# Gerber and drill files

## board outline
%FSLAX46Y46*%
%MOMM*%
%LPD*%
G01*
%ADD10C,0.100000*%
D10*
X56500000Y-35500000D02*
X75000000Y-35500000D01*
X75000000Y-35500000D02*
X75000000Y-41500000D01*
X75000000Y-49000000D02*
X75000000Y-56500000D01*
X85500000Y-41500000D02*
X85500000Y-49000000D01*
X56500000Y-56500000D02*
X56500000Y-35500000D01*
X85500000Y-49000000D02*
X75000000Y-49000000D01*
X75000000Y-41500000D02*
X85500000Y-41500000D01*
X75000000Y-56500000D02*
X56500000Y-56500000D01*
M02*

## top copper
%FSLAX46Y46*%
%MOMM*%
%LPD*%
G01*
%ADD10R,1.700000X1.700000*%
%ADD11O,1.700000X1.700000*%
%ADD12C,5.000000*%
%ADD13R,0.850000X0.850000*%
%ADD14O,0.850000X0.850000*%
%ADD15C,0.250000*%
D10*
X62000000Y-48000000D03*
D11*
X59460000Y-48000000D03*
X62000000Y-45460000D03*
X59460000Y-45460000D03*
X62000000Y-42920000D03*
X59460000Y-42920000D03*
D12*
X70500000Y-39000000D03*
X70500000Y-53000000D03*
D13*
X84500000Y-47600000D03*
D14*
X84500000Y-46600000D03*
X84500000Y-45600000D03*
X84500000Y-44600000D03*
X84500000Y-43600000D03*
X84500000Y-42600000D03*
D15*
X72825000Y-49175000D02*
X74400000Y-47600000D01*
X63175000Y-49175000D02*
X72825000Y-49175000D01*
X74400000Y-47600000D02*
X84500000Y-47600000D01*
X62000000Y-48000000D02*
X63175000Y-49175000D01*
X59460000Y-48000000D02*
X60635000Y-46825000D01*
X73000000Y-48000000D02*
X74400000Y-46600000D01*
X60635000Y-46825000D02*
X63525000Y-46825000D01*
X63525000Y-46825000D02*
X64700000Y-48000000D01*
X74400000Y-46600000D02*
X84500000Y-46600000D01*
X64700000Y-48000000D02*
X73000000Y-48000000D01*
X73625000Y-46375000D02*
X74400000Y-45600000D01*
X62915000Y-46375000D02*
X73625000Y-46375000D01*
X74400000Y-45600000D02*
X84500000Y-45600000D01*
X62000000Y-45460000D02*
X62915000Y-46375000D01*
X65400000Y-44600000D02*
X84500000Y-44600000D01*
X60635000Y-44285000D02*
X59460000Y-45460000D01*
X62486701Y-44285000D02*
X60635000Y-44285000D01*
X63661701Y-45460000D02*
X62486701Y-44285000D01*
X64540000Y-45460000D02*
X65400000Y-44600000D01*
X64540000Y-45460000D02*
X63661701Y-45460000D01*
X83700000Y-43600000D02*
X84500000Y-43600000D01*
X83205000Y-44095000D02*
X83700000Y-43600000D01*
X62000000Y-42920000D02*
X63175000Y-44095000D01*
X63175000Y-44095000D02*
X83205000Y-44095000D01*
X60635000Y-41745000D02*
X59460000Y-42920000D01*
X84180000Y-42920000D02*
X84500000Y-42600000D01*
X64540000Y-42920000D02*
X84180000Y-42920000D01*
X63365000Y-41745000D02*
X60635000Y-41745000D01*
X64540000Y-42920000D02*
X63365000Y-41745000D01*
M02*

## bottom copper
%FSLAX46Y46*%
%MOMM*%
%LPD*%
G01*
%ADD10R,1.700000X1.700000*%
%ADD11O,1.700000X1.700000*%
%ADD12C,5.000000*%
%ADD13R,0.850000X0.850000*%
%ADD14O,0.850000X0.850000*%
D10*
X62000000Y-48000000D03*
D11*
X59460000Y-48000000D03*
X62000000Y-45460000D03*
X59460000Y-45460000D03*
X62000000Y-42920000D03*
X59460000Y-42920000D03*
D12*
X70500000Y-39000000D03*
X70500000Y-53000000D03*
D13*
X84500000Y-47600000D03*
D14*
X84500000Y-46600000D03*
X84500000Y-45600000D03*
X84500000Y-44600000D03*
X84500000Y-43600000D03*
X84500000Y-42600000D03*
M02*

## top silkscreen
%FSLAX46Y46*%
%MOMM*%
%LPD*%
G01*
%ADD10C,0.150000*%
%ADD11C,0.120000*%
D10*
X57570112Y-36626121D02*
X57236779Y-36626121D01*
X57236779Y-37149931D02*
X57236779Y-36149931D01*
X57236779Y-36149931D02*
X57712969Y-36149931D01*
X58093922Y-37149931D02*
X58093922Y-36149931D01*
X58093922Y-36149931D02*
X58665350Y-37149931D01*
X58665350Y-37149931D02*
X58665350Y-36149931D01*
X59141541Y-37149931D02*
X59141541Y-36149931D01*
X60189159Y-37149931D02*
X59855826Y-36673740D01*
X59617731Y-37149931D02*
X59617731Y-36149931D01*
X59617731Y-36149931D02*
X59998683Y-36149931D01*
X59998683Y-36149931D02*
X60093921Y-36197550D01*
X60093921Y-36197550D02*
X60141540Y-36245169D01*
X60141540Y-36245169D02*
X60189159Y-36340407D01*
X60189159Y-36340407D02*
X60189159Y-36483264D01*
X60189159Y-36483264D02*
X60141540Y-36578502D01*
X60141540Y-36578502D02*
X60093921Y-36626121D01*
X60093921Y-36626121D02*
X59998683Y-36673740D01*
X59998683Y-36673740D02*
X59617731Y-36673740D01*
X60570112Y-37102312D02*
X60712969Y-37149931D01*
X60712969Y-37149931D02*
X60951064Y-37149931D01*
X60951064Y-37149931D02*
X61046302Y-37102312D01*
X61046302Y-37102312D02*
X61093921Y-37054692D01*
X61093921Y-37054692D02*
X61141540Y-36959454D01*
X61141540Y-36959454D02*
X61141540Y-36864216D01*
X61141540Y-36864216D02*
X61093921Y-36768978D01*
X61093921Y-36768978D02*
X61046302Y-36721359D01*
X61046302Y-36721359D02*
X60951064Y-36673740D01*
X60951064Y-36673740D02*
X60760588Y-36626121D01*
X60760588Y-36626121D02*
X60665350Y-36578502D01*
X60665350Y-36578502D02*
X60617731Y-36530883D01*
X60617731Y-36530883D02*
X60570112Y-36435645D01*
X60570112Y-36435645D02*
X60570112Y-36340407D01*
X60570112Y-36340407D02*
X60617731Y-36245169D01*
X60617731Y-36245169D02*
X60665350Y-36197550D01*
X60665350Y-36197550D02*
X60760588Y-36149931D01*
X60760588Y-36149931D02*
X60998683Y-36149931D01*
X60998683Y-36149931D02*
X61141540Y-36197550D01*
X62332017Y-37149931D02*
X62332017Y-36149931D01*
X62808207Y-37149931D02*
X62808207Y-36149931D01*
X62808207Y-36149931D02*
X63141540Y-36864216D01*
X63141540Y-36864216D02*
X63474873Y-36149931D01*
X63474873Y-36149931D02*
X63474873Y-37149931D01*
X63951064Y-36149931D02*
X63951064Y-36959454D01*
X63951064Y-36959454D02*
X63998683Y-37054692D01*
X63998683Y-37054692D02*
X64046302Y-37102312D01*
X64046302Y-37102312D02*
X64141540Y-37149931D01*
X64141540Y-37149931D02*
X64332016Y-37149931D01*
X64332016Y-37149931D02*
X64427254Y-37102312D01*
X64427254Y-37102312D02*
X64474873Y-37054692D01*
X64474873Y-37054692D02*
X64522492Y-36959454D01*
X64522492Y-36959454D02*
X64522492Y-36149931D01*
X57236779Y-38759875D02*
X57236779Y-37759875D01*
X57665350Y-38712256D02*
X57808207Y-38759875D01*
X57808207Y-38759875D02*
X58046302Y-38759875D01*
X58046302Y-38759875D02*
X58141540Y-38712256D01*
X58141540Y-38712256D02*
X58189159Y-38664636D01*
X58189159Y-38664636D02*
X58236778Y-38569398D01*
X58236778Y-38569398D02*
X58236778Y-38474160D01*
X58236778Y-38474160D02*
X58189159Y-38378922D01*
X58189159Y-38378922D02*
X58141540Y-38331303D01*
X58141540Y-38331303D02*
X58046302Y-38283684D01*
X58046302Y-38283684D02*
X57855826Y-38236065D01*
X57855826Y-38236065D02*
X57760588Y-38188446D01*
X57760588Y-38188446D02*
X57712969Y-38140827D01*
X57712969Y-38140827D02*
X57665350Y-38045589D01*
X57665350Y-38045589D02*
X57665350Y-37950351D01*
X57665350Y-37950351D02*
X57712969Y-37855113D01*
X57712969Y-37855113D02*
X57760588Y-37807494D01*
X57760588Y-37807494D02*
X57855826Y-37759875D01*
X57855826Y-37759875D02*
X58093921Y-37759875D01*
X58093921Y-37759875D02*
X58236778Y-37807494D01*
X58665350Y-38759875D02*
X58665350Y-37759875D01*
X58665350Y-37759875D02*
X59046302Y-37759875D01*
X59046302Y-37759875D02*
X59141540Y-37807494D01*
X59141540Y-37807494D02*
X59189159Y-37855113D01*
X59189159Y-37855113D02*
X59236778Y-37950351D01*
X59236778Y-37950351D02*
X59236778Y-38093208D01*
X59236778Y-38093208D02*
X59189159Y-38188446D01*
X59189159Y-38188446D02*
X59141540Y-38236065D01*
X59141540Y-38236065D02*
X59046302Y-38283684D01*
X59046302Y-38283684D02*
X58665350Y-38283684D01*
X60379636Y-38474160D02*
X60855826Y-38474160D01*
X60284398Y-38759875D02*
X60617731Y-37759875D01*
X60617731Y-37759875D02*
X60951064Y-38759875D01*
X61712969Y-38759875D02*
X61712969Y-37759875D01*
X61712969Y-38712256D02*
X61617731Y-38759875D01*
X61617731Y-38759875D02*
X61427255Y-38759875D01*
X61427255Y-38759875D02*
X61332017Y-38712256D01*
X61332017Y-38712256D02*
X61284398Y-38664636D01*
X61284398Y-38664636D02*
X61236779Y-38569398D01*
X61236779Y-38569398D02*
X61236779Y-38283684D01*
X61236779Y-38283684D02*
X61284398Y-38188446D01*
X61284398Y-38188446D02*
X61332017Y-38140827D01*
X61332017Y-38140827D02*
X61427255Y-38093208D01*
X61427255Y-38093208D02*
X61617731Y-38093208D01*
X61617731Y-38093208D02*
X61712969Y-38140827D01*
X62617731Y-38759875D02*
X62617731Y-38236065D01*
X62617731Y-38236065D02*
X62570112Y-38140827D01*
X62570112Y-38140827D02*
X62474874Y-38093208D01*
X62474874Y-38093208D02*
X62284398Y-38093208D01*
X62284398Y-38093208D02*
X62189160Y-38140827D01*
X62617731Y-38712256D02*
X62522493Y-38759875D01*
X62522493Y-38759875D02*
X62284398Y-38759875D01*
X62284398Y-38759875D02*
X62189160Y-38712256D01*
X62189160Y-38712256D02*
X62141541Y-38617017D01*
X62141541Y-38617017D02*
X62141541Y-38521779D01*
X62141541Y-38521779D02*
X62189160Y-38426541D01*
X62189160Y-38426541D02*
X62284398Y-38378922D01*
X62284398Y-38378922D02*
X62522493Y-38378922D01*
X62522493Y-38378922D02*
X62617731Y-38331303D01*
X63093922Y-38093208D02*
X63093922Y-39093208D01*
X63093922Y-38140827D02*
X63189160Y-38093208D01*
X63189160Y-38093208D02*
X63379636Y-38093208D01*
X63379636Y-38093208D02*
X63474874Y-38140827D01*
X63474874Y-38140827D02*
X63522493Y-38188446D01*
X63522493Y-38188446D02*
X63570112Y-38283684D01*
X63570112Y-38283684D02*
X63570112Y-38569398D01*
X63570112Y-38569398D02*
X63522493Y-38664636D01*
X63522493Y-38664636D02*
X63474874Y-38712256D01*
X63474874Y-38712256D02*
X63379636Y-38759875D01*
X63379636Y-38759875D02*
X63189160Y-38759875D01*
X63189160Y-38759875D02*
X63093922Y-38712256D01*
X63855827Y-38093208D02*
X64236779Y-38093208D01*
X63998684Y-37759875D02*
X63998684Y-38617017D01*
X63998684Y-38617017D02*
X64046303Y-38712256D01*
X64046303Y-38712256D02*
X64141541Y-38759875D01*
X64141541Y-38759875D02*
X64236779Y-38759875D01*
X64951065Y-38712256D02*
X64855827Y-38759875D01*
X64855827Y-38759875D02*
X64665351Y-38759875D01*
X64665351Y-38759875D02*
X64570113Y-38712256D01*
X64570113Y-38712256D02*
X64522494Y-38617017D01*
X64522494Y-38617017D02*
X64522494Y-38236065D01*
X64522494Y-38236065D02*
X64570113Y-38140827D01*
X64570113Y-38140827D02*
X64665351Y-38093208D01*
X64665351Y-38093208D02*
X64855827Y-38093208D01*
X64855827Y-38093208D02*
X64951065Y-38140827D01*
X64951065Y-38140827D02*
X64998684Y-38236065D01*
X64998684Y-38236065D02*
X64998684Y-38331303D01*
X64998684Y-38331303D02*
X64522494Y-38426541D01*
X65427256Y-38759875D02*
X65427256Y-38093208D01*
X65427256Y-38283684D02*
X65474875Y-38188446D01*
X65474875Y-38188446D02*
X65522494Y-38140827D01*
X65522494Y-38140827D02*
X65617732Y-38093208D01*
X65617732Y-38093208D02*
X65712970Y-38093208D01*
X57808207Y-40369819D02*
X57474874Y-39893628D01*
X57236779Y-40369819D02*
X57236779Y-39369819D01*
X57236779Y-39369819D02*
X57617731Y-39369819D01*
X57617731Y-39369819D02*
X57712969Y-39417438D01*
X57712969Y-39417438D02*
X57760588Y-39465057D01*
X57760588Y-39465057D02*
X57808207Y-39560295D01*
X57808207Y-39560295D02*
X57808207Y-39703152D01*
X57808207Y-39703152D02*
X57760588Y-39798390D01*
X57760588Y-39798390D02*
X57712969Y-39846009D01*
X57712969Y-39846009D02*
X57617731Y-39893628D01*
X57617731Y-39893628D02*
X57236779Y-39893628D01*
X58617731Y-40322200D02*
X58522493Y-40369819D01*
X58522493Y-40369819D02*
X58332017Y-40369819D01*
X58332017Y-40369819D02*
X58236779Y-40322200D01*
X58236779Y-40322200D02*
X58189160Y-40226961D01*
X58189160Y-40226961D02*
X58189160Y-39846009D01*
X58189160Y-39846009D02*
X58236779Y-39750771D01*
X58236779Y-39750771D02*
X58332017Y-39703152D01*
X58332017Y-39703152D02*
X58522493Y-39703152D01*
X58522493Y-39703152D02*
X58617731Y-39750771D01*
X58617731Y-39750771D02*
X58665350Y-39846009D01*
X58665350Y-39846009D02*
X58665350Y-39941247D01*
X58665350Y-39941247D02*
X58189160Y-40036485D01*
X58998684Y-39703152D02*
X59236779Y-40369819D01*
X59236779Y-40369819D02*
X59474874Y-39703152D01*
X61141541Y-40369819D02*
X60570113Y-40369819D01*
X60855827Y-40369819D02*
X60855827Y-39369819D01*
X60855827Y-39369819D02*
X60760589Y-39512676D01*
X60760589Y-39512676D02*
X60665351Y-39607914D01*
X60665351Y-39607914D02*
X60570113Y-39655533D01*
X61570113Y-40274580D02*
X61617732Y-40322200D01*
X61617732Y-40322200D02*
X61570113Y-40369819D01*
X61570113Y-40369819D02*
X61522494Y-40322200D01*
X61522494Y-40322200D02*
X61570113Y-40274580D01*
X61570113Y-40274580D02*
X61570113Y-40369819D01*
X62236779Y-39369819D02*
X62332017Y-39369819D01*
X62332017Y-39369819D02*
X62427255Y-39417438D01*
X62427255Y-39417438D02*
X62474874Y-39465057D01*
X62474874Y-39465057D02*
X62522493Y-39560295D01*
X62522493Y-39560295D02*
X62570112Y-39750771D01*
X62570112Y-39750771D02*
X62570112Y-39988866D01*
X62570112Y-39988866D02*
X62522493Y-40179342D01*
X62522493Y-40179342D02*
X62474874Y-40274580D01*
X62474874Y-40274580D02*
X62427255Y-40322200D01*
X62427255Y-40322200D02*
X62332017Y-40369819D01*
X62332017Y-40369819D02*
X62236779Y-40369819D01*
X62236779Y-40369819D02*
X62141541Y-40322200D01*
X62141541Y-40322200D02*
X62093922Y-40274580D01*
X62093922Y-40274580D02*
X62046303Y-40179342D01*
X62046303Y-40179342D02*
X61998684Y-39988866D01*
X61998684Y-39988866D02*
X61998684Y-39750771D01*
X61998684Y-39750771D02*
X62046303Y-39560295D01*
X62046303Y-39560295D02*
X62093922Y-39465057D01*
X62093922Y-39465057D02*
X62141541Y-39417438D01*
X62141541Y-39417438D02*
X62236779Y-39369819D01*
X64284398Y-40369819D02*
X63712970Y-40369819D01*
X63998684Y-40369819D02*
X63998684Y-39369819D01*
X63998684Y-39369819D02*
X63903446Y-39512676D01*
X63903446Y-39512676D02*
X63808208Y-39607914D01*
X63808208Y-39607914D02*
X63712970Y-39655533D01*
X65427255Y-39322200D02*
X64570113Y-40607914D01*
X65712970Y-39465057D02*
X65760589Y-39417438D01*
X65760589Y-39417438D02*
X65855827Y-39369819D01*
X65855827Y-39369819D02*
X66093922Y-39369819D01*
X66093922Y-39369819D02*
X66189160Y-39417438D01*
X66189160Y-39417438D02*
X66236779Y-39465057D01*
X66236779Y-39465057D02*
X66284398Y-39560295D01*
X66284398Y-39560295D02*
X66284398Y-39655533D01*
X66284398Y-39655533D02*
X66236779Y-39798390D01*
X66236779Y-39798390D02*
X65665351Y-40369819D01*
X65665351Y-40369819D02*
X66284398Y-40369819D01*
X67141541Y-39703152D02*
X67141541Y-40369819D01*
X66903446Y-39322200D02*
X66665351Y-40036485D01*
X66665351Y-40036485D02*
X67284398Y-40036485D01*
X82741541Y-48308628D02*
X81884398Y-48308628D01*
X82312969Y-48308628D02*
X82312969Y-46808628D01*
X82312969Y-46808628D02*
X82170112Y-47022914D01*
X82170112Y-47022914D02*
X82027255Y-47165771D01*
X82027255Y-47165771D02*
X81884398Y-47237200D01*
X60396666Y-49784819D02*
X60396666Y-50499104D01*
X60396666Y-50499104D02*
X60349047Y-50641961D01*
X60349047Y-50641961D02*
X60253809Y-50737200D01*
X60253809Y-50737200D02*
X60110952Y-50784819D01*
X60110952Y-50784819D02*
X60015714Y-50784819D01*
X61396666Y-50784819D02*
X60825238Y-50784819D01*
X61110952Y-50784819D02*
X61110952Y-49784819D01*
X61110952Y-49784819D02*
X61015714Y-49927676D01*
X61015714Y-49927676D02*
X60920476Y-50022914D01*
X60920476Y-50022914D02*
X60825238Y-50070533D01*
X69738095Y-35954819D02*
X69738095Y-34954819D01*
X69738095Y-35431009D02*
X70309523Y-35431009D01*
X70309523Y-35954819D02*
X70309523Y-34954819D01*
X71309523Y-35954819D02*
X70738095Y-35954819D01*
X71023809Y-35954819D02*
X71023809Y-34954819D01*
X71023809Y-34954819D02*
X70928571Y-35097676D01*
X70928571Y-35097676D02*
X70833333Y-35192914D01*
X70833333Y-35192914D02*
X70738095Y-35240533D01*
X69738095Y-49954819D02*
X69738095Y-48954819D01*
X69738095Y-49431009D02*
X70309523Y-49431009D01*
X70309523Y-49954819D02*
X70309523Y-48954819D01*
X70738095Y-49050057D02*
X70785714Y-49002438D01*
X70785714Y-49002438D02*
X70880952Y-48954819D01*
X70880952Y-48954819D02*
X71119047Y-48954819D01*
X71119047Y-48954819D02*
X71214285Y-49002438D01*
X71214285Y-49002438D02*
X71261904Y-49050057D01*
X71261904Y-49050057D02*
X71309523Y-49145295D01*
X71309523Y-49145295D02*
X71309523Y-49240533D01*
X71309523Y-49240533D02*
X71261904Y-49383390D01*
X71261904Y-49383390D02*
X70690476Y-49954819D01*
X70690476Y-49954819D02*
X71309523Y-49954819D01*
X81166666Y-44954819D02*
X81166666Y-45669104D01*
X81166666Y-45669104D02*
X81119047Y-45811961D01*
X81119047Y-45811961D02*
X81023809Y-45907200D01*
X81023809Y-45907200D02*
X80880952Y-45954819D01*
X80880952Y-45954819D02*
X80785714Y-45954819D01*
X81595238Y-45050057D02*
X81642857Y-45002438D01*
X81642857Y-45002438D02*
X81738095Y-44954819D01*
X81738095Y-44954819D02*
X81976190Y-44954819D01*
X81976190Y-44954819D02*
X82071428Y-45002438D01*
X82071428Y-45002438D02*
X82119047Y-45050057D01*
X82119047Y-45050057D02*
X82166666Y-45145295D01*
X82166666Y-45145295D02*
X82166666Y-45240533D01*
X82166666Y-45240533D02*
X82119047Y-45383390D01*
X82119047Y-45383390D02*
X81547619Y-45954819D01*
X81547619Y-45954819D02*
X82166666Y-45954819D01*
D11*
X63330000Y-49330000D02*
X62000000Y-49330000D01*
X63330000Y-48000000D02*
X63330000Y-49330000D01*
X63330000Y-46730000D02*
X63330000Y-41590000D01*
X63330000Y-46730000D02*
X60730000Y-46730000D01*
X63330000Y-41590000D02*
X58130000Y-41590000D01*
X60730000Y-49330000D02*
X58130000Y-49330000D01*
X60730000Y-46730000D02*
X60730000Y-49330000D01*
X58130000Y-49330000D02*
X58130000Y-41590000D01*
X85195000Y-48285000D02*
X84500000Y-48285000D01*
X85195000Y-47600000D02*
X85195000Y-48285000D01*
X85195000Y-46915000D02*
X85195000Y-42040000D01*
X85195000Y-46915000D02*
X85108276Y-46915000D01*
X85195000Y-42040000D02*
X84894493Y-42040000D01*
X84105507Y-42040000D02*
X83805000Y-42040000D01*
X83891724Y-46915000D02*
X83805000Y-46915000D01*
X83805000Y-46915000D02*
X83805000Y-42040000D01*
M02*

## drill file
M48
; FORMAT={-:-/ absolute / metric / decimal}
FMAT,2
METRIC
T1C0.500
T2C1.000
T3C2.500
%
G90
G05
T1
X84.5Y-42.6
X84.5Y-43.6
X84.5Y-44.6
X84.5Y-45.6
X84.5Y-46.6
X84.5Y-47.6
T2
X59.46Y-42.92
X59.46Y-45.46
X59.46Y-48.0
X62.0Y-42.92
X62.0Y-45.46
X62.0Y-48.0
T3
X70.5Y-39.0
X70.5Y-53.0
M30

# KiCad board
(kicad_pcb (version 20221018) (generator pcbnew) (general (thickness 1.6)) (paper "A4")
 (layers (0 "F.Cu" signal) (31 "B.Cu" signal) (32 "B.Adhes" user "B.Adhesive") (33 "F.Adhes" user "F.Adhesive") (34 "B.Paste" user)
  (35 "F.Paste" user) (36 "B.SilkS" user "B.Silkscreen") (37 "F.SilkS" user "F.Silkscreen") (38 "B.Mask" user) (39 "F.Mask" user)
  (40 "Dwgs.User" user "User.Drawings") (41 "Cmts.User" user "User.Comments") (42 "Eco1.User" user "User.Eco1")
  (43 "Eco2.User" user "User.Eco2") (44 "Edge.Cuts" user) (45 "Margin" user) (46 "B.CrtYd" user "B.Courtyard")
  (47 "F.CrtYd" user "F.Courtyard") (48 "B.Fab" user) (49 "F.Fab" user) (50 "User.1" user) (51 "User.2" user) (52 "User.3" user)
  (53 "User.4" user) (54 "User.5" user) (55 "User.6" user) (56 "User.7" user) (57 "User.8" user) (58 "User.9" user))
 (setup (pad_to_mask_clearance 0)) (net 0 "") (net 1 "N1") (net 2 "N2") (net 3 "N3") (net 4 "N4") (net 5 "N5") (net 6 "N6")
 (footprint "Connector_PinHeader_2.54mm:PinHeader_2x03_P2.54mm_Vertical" (layer "F.Cu") (at 62 48 180)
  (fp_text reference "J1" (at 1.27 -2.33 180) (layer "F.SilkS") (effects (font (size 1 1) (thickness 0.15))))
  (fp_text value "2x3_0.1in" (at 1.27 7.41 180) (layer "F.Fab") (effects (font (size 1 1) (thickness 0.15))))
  (fp_line (start -1.33 -1.33) (end 0 -1.33) (stroke (width 0.12) (type solid)) (layer "F.SilkS"))
  (fp_line (start -1.33 0) (end -1.33 -1.33) (stroke (width 0.12) (type solid)) (layer "F.SilkS"))
  (fp_line (start -1.33 1.27) (end -1.33 6.41) (stroke (width 0.12) (type solid)) (layer "F.SilkS"))
  (fp_line (start -1.33 1.27) (end 1.27 1.27) (stroke (width 0.12) (type solid)) (layer "F.SilkS"))
  (fp_line (start -1.33 6.41) (end 3.87 6.41) (stroke (width 0.12) (type solid)) (layer "F.SilkS"))
  (fp_line (start 1.27 -1.33) (end 3.87 -1.33) (stroke (width 0.12) (type solid)) (layer "F.SilkS"))
  (fp_line (start 1.27 1.27) (end 1.27 -1.33) (stroke (width 0.12) (type solid)) (layer "F.SilkS"))
  (fp_line (start 3.87 -1.33) (end 3.87 6.41) (stroke (width 0.12) (type solid)) (layer "F.SilkS"))
  (pad "1" thru_hole rect (at 0 0 180) (size 1.7 1.7) (drill 1) (layers "*.Cu" "*.Mask") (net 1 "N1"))
  (pad "2" thru_hole oval (at 2.54 0 180) (size 1.7 1.7) (drill 1) (layers "*.Cu" "*.Mask") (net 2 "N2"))
  (pad "3" thru_hole oval (at 0 2.54 180) (size 1.7 1.7) (drill 1) (layers "*.Cu" "*.Mask") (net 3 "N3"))
  (pad "4" thru_hole oval (at 2.54 2.54 180) (size 1.7 1.7) (drill 1) (layers "*.Cu" "*.Mask") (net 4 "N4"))
  (pad "5" thru_hole oval (at 0 5.08 180) (size 1.7 1.7) (drill 1) (layers "*.Cu" "*.Mask") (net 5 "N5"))
  (pad "6" thru_hole oval (at 2.54 5.08 180) (size 1.7 1.7) (drill 1) (layers "*.Cu" "*.Mask") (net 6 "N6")))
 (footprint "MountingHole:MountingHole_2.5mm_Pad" (layer "F.Cu") (at 70.5 39)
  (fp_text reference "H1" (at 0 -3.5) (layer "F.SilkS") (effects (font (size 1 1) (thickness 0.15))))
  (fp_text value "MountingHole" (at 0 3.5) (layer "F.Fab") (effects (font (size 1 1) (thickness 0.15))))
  (pad "1" thru_hole circle (at 0 0) (size 5 5) (drill 2.5) (layers "*.Cu" "*.Mask")))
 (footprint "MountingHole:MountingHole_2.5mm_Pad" (layer "F.Cu") (at 70.5 53)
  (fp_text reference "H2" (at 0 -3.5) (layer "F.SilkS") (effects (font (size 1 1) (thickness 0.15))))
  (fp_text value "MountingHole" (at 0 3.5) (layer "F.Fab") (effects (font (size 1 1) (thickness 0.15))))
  (pad "1" thru_hole circle (at 0 0) (size 5 5) (drill 2.5) (layers "*.Cu" "*.Mask")))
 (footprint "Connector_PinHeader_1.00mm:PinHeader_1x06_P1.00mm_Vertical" (layer "F.Cu") (at 84.5 47.6 180)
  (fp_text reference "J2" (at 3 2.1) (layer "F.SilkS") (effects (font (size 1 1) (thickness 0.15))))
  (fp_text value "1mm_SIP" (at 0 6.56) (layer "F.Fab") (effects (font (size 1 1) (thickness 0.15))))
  (fp_line (start -0.695 -0.685) (end 0 -0.685) (stroke (width 0.12) (type solid)) (layer "F.SilkS"))
  (fp_line (start -0.695 0) (end -0.695 -0.685) (stroke (width 0.12) (type solid)) (layer "F.SilkS"))
  (fp_line (start -0.695 0.685) (end -0.695 5.56) (stroke (width 0.12) (type solid)) (layer "F.SilkS"))
  (fp_line (start -0.695 0.685) (end -0.608276 0.685) (stroke (width 0.12) (type solid)) (layer "F.SilkS"))
  (fp_line (start -0.695 5.56) (end -0.394493 5.56) (stroke (width 0.12) (type solid)) (layer "F.SilkS"))
  (fp_line (start 0.394493 5.56) (end 0.695 5.56) (stroke (width 0.12) (type solid)) (layer "F.SilkS"))
  (fp_line (start 0.608276 0.685) (end 0.695 0.685) (stroke (width 0.12) (type solid)) (layer "F.SilkS"))
  (fp_line (start 0.695 0.685) (end 0.695 5.56) (stroke (width 0.12) (type solid)) (layer "F.SilkS"))
  (pad "1" thru_hole rect (at 0 0 180) (size 0.85 0.85) (drill 0.5) (layers "*.Cu" "*.Mask") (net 1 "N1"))
  (pad "2" thru_hole oval (at 0 1 180) (size 0.85 0.85) (drill 0.5) (layers "*.Cu" "*.Mask") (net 2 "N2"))
  (pad "3" thru_hole oval (at 0 2 180) (size 0.85 0.85) (drill 0.5) (layers "*.Cu" "*.Mask") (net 3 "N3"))
  (pad "4" thru_hole oval (at 0 3 180) (size 0.85 0.85) (drill 0.5) (layers "*.Cu" "*.Mask") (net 4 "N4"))
  (pad "5" thru_hole oval (at 0 4 180) (size 0.85 0.85) (drill 0.5) (layers "*.Cu" "*.Mask") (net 5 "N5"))
  (pad "6" thru_hole oval (at 0 5 180) (size 0.85 0.85) (drill 0.5) (layers "*.Cu" "*.Mask") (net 6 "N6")))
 (gr_line (start 56.5 35.5) (end 75 35.5) (stroke (width 0.1) (type default)) (layer "Edge.Cuts"))
 (gr_line (start 75 35.5) (end 75 41.5) (stroke (width 0.1) (type default)) (layer "Edge.Cuts"))
 (gr_line (start 75 49) (end 75 56.5) (stroke (width 0.1) (type default)) (layer "Edge.Cuts"))
 (gr_line (start 85.5 41.5) (end 85.5 49) (stroke (width 0.1) (type default)) (layer "Edge.Cuts"))
 (gr_line (start 56.5 56.5) (end 56.5 35.5) (stroke (width 0.1) (type default)) (layer "Edge.Cuts"))
 (gr_line (start 85.5 49) (end 75 49) (stroke (width 0.1) (type default)) (layer "Edge.Cuts"))
 (gr_line (start 75 41.5) (end 85.5 41.5) (stroke (width 0.1) (type default)) (layer "Edge.Cuts"))
 (gr_line (start 75 56.5) (end 56.5 56.5) (stroke (width 0.1) (type default)) (layer "Edge.Cuts"))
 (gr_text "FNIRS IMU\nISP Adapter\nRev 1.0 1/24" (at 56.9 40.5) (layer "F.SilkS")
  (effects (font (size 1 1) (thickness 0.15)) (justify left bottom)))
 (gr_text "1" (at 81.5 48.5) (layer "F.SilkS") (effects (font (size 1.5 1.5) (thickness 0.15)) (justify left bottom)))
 (segment (start 72.825 49.175) (end 74.4 47.6) (width 0.25) (layer "F.Cu") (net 1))
 (segment (start 63.175 49.175) (end 72.825 49.175) (width 0.25) (layer "F.Cu") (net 1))
 (segment (start 74.4 47.6) (end 84.5 47.6) (width 0.25) (layer "F.Cu") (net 1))
 (segment (start 62 48) (end 63.175 49.175) (width 0.25) (layer "F.Cu") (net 1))
 (segment (start 59.46 48) (end 60.635 46.825) (width 0.25) (layer "F.Cu") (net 2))
 (segment (start 73 48) (end 74.4 46.6) (width 0.25) (layer "F.Cu") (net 2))
 (segment (start 60.635 46.825) (end 63.525 46.825) (width 0.25) (layer "F.Cu") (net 2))
 (segment (start 63.525 46.825) (end 64.7 48) (width 0.25) (layer "F.Cu") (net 2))
 (segment (start 74.4 46.6) (end 84.5 46.6) (width 0.25) (layer "F.Cu") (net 2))
 (segment (start 64.7 48) (end 73 48) (width 0.25) (layer "F.Cu") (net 2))
 (segment (start 73.625 46.375) (end 74.4 45.6) (width 0.25) (layer "F.Cu") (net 3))
 (segment (start 62.915 46.375) (end 73.625 46.375) (width 0.25) (layer "F.Cu") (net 3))
 (segment (start 74.4 45.6) (end 84.5 45.6) (width 0.25) (layer "F.Cu") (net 3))
 (segment (start 62 45.46) (end 62.915 46.375) (width 0.25) (layer "F.Cu") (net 3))
 (segment (start 65.4 44.6) (end 84.5 44.6) (width 0.25) (layer "F.Cu") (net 4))
 (segment (start 60.635 44.285) (end 59.46 45.46) (width 0.25) (layer "F.Cu") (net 4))
 (segment (start 62.486701 44.285) (end 60.635 44.285) (width 0.25) (layer "F.Cu") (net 4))
 (segment (start 63.661701 45.46) (end 62.486701 44.285) (width 0.25) (layer "F.Cu") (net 4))
 (segment (start 64.54 45.46) (end 65.4 44.6) (width 0.25) (layer "F.Cu") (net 4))
 (segment (start 64.54 45.46) (end 63.661701 45.46) (width 0.25) (layer "F.Cu") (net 4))
 (segment (start 83.7 43.6) (end 84.5 43.6) (width 0.25) (layer "F.Cu") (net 5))
 (segment (start 83.205 44.095) (end 83.7 43.6) (width 0.25) (layer "F.Cu") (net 5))
 (segment (start 62 42.92) (end 63.175 44.095) (width 0.25) (layer "F.Cu") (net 5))
 (segment (start 63.175 44.095) (end 83.205 44.095) (width 0.25) (layer "F.Cu") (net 5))
 (segment (start 60.635 41.745) (end 59.46 42.92) (width 0.25) (layer "F.Cu") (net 6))
 (segment (start 84.18 42.92) (end 84.5 42.6) (width 0.25) (layer "F.Cu") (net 6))
 (segment (start 64.54 42.92) (end 84.18 42.92) (width 0.25) (layer "F.Cu") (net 6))
 (segment (start 63.365 41.745) (end 60.635 41.745) (width 0.25) (layer "F.Cu") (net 6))
 (segment (start 64.54 42.92) (end 63.365 41.745) (width 0.25) (layer "F.Cu") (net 6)))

